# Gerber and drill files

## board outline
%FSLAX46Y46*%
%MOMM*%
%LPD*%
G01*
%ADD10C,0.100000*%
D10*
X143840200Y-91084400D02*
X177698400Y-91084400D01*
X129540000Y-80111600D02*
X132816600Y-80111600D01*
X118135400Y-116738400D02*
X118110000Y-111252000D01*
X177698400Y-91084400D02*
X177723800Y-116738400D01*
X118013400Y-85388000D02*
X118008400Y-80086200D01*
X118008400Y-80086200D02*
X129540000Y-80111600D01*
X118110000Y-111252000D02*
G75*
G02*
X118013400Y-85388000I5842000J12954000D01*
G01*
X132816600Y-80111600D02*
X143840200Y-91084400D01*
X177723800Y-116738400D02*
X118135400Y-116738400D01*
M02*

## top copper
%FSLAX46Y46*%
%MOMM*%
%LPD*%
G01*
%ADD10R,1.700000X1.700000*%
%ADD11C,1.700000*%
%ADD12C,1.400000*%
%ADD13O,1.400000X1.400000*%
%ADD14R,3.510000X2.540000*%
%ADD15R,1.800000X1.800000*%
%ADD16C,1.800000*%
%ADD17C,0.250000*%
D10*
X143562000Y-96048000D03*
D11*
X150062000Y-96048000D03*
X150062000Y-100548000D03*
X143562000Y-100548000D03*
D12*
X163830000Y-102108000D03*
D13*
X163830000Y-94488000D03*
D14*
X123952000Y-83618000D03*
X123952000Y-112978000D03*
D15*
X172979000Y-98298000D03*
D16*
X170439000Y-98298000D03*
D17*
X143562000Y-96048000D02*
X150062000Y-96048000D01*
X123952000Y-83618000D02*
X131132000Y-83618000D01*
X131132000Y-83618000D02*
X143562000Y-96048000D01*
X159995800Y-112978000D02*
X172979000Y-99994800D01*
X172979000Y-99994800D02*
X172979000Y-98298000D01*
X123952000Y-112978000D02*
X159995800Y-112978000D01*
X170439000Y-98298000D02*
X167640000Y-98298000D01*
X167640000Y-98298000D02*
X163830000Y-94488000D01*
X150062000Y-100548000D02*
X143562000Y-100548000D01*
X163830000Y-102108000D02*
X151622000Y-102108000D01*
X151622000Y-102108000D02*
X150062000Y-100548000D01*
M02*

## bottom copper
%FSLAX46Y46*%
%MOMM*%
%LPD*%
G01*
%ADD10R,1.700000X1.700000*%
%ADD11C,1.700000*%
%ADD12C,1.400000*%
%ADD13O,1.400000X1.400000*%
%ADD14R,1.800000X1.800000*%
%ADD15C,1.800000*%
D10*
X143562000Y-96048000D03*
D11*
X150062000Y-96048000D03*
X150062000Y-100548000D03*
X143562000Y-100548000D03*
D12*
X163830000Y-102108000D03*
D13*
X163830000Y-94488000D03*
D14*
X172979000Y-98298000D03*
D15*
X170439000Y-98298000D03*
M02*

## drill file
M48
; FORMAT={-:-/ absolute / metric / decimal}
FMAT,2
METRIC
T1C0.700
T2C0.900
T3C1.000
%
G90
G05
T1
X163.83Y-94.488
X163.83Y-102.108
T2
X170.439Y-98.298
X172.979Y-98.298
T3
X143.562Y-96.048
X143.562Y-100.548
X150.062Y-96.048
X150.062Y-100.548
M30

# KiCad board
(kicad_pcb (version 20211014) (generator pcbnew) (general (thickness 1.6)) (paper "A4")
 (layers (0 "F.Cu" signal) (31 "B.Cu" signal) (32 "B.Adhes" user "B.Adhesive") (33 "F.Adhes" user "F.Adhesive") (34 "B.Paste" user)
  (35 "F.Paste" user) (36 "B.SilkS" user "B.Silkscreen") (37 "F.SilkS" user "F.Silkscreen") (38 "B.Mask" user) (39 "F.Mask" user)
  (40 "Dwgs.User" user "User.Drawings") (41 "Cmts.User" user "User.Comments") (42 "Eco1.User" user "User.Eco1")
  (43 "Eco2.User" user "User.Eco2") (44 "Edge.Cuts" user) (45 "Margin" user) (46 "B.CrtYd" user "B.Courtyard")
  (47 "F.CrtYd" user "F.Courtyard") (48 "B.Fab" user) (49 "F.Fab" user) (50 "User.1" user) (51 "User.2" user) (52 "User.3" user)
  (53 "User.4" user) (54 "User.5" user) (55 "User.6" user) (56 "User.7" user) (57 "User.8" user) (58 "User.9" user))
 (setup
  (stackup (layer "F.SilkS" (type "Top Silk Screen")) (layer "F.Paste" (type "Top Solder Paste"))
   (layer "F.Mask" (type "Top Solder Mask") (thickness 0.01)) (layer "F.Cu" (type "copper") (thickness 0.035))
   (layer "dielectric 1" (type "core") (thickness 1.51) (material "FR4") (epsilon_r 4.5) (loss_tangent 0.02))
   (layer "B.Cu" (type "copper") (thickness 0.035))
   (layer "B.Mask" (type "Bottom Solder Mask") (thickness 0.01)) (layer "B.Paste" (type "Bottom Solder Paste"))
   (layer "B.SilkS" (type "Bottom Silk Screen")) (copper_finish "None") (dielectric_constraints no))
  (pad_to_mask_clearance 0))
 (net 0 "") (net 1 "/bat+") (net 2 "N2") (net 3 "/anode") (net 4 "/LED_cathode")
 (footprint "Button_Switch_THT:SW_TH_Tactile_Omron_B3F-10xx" (layer "F.Cu") (at 143.562 96.048)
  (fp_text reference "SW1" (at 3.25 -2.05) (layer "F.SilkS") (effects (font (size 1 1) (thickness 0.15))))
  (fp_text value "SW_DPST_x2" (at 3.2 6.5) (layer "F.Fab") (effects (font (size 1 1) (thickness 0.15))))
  (pad "1" thru_hole rect (at 0 0) (size 1.7 1.7) (drill 1) (layers *.Cu *.Mask) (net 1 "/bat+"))
  (pad "1" thru_hole circle (at 6.5 0) (size 1.7 1.7) (drill 1) (layers *.Cu *.Mask) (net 1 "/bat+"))
  (pad "2" thru_hole circle (at 6.5 4.5) (size 1.7 1.7) (drill 1) (layers *.Cu *.Mask) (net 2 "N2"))
  (pad "2" thru_hole circle (at 0 4.5) (size 1.7 1.7) (drill 1) (layers *.Cu *.Mask) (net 2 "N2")))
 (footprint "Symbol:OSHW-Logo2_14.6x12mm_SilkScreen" (layer "F.Cu") (at 169.3418 110.1852)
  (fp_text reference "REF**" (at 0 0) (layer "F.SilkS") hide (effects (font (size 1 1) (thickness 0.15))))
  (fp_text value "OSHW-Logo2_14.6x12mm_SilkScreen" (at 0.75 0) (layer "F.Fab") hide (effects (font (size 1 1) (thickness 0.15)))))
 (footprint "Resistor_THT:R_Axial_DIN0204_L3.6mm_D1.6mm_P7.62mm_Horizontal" (layer "F.Cu") (at 163.83 102.108 90)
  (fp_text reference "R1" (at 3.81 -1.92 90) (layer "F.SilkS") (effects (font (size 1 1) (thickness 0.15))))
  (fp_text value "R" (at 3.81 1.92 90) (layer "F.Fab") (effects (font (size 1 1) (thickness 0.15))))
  (pad "1" thru_hole circle (at 0 0 90) (size 1.4 1.4) (drill 0.7) (layers *.Cu *.Mask) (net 2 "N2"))
  (pad "2" thru_hole oval (at 7.62 0 90) (size 1.4 1.4) (drill 0.7) (layers *.Cu *.Mask) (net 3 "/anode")))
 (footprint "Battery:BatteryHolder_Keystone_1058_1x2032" (layer "F.Cu") (at 123.952 98.298 -90)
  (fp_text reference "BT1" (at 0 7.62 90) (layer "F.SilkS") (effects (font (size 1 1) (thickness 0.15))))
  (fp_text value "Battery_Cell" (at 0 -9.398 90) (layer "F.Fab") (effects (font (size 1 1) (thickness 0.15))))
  (pad "1" smd rect (at -14.68 0 270) (size 2.54 3.51) (layers "F.Cu" "F.Paste" "F.Mask") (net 1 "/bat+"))
  (pad "2" smd rect (at 14.68 0 270) (size 2.54 3.51) (layers "F.Cu" "F.Paste" "F.Mask") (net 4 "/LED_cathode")))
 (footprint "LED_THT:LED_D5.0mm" (layer "F.Cu") (at 172.979 98.298 180)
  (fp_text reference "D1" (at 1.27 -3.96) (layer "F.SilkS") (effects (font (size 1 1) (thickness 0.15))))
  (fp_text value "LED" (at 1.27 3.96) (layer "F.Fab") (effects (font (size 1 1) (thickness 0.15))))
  (pad "1" thru_hole rect (at 0 0 180) (size 1.8 1.8) (drill 0.9) (layers *.Cu *.Mask) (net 4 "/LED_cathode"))
  (pad "2" thru_hole circle (at 2.54 0 180) (size 1.8 1.8) (drill 0.9) (layers *.Cu *.Mask) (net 3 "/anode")))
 (gr_line (start 143.8402 91.0844) (end 177.6984 91.0844) (layer "Edge.Cuts") (width 0.1))
 (gr_line (start 129.54 80.1116) (end 132.8166 80.1116) (layer "Edge.Cuts") (width 0.1))
 (gr_line (start 118.1354 116.7384) (end 118.11 111.252) (layer "Edge.Cuts") (width 0.1))
 (gr_line (start 177.6984 91.0844) (end 177.7238 116.7384) (layer "Edge.Cuts") (width 0.1))
 (gr_line (start 118.0134 85.388) (end 118.0084 80.0862) (layer "Edge.Cuts") (width 0.1))
 (gr_line (start 118.0084 80.0862) (end 129.54 80.1116) (layer "Edge.Cuts") (width 0.1))
 (gr_arc (start 118.11 111.252) (mid 109.741713 98.351074) (end 118.0134 85.388) (layer "Edge.Cuts") (width 0.1))
 (gr_line (start 132.8166 80.1116) (end 143.8402 91.0844) (layer "Edge.Cuts") (width 0.1))
 (gr_line (start 177.7238 116.7384) (end 118.1354 116.7384) (layer "Edge.Cuts") (width 0.1))
 (segment (start 143.562 96.048) (end 150.062 96.048) (width 0.25) (layer "F.Cu") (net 1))
 (segment (start 123.952 83.618) (end 131.132 83.618) (width 0.25) (layer "F.Cu") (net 1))
 (segment (start 131.132 83.618) (end 143.562 96.048) (width 0.25) (layer "F.Cu") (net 1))
 (segment (start 159.9958 112.978) (end 172.979 99.9948) (width 0.25) (layer "F.Cu") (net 4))
 (segment (start 172.979 99.9948) (end 172.979 98.298) (width 0.25) (layer "F.Cu") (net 4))
 (segment (start 123.952 112.978) (end 159.9958 112.978) (width 0.25) (layer "F.Cu") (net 4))
 (segment (start 170.439 98.298) (end 167.64 98.298) (width 0.25) (layer "F.Cu") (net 3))
 (segment (start 167.64 98.298) (end 163.83 94.488) (width 0.25) (layer "F.Cu") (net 3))
 (segment (start 150.062 100.548) (end 143.562 100.548) (width 0.25) (layer "F.Cu") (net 2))
 (segment (start 163.83 102.108) (end 151.622 102.108) (width 0.25) (layer "F.Cu") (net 2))
 (segment (start 151.622 102.108) (end 150.062 100.548) (width 0.25) (layer "F.Cu") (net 2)))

